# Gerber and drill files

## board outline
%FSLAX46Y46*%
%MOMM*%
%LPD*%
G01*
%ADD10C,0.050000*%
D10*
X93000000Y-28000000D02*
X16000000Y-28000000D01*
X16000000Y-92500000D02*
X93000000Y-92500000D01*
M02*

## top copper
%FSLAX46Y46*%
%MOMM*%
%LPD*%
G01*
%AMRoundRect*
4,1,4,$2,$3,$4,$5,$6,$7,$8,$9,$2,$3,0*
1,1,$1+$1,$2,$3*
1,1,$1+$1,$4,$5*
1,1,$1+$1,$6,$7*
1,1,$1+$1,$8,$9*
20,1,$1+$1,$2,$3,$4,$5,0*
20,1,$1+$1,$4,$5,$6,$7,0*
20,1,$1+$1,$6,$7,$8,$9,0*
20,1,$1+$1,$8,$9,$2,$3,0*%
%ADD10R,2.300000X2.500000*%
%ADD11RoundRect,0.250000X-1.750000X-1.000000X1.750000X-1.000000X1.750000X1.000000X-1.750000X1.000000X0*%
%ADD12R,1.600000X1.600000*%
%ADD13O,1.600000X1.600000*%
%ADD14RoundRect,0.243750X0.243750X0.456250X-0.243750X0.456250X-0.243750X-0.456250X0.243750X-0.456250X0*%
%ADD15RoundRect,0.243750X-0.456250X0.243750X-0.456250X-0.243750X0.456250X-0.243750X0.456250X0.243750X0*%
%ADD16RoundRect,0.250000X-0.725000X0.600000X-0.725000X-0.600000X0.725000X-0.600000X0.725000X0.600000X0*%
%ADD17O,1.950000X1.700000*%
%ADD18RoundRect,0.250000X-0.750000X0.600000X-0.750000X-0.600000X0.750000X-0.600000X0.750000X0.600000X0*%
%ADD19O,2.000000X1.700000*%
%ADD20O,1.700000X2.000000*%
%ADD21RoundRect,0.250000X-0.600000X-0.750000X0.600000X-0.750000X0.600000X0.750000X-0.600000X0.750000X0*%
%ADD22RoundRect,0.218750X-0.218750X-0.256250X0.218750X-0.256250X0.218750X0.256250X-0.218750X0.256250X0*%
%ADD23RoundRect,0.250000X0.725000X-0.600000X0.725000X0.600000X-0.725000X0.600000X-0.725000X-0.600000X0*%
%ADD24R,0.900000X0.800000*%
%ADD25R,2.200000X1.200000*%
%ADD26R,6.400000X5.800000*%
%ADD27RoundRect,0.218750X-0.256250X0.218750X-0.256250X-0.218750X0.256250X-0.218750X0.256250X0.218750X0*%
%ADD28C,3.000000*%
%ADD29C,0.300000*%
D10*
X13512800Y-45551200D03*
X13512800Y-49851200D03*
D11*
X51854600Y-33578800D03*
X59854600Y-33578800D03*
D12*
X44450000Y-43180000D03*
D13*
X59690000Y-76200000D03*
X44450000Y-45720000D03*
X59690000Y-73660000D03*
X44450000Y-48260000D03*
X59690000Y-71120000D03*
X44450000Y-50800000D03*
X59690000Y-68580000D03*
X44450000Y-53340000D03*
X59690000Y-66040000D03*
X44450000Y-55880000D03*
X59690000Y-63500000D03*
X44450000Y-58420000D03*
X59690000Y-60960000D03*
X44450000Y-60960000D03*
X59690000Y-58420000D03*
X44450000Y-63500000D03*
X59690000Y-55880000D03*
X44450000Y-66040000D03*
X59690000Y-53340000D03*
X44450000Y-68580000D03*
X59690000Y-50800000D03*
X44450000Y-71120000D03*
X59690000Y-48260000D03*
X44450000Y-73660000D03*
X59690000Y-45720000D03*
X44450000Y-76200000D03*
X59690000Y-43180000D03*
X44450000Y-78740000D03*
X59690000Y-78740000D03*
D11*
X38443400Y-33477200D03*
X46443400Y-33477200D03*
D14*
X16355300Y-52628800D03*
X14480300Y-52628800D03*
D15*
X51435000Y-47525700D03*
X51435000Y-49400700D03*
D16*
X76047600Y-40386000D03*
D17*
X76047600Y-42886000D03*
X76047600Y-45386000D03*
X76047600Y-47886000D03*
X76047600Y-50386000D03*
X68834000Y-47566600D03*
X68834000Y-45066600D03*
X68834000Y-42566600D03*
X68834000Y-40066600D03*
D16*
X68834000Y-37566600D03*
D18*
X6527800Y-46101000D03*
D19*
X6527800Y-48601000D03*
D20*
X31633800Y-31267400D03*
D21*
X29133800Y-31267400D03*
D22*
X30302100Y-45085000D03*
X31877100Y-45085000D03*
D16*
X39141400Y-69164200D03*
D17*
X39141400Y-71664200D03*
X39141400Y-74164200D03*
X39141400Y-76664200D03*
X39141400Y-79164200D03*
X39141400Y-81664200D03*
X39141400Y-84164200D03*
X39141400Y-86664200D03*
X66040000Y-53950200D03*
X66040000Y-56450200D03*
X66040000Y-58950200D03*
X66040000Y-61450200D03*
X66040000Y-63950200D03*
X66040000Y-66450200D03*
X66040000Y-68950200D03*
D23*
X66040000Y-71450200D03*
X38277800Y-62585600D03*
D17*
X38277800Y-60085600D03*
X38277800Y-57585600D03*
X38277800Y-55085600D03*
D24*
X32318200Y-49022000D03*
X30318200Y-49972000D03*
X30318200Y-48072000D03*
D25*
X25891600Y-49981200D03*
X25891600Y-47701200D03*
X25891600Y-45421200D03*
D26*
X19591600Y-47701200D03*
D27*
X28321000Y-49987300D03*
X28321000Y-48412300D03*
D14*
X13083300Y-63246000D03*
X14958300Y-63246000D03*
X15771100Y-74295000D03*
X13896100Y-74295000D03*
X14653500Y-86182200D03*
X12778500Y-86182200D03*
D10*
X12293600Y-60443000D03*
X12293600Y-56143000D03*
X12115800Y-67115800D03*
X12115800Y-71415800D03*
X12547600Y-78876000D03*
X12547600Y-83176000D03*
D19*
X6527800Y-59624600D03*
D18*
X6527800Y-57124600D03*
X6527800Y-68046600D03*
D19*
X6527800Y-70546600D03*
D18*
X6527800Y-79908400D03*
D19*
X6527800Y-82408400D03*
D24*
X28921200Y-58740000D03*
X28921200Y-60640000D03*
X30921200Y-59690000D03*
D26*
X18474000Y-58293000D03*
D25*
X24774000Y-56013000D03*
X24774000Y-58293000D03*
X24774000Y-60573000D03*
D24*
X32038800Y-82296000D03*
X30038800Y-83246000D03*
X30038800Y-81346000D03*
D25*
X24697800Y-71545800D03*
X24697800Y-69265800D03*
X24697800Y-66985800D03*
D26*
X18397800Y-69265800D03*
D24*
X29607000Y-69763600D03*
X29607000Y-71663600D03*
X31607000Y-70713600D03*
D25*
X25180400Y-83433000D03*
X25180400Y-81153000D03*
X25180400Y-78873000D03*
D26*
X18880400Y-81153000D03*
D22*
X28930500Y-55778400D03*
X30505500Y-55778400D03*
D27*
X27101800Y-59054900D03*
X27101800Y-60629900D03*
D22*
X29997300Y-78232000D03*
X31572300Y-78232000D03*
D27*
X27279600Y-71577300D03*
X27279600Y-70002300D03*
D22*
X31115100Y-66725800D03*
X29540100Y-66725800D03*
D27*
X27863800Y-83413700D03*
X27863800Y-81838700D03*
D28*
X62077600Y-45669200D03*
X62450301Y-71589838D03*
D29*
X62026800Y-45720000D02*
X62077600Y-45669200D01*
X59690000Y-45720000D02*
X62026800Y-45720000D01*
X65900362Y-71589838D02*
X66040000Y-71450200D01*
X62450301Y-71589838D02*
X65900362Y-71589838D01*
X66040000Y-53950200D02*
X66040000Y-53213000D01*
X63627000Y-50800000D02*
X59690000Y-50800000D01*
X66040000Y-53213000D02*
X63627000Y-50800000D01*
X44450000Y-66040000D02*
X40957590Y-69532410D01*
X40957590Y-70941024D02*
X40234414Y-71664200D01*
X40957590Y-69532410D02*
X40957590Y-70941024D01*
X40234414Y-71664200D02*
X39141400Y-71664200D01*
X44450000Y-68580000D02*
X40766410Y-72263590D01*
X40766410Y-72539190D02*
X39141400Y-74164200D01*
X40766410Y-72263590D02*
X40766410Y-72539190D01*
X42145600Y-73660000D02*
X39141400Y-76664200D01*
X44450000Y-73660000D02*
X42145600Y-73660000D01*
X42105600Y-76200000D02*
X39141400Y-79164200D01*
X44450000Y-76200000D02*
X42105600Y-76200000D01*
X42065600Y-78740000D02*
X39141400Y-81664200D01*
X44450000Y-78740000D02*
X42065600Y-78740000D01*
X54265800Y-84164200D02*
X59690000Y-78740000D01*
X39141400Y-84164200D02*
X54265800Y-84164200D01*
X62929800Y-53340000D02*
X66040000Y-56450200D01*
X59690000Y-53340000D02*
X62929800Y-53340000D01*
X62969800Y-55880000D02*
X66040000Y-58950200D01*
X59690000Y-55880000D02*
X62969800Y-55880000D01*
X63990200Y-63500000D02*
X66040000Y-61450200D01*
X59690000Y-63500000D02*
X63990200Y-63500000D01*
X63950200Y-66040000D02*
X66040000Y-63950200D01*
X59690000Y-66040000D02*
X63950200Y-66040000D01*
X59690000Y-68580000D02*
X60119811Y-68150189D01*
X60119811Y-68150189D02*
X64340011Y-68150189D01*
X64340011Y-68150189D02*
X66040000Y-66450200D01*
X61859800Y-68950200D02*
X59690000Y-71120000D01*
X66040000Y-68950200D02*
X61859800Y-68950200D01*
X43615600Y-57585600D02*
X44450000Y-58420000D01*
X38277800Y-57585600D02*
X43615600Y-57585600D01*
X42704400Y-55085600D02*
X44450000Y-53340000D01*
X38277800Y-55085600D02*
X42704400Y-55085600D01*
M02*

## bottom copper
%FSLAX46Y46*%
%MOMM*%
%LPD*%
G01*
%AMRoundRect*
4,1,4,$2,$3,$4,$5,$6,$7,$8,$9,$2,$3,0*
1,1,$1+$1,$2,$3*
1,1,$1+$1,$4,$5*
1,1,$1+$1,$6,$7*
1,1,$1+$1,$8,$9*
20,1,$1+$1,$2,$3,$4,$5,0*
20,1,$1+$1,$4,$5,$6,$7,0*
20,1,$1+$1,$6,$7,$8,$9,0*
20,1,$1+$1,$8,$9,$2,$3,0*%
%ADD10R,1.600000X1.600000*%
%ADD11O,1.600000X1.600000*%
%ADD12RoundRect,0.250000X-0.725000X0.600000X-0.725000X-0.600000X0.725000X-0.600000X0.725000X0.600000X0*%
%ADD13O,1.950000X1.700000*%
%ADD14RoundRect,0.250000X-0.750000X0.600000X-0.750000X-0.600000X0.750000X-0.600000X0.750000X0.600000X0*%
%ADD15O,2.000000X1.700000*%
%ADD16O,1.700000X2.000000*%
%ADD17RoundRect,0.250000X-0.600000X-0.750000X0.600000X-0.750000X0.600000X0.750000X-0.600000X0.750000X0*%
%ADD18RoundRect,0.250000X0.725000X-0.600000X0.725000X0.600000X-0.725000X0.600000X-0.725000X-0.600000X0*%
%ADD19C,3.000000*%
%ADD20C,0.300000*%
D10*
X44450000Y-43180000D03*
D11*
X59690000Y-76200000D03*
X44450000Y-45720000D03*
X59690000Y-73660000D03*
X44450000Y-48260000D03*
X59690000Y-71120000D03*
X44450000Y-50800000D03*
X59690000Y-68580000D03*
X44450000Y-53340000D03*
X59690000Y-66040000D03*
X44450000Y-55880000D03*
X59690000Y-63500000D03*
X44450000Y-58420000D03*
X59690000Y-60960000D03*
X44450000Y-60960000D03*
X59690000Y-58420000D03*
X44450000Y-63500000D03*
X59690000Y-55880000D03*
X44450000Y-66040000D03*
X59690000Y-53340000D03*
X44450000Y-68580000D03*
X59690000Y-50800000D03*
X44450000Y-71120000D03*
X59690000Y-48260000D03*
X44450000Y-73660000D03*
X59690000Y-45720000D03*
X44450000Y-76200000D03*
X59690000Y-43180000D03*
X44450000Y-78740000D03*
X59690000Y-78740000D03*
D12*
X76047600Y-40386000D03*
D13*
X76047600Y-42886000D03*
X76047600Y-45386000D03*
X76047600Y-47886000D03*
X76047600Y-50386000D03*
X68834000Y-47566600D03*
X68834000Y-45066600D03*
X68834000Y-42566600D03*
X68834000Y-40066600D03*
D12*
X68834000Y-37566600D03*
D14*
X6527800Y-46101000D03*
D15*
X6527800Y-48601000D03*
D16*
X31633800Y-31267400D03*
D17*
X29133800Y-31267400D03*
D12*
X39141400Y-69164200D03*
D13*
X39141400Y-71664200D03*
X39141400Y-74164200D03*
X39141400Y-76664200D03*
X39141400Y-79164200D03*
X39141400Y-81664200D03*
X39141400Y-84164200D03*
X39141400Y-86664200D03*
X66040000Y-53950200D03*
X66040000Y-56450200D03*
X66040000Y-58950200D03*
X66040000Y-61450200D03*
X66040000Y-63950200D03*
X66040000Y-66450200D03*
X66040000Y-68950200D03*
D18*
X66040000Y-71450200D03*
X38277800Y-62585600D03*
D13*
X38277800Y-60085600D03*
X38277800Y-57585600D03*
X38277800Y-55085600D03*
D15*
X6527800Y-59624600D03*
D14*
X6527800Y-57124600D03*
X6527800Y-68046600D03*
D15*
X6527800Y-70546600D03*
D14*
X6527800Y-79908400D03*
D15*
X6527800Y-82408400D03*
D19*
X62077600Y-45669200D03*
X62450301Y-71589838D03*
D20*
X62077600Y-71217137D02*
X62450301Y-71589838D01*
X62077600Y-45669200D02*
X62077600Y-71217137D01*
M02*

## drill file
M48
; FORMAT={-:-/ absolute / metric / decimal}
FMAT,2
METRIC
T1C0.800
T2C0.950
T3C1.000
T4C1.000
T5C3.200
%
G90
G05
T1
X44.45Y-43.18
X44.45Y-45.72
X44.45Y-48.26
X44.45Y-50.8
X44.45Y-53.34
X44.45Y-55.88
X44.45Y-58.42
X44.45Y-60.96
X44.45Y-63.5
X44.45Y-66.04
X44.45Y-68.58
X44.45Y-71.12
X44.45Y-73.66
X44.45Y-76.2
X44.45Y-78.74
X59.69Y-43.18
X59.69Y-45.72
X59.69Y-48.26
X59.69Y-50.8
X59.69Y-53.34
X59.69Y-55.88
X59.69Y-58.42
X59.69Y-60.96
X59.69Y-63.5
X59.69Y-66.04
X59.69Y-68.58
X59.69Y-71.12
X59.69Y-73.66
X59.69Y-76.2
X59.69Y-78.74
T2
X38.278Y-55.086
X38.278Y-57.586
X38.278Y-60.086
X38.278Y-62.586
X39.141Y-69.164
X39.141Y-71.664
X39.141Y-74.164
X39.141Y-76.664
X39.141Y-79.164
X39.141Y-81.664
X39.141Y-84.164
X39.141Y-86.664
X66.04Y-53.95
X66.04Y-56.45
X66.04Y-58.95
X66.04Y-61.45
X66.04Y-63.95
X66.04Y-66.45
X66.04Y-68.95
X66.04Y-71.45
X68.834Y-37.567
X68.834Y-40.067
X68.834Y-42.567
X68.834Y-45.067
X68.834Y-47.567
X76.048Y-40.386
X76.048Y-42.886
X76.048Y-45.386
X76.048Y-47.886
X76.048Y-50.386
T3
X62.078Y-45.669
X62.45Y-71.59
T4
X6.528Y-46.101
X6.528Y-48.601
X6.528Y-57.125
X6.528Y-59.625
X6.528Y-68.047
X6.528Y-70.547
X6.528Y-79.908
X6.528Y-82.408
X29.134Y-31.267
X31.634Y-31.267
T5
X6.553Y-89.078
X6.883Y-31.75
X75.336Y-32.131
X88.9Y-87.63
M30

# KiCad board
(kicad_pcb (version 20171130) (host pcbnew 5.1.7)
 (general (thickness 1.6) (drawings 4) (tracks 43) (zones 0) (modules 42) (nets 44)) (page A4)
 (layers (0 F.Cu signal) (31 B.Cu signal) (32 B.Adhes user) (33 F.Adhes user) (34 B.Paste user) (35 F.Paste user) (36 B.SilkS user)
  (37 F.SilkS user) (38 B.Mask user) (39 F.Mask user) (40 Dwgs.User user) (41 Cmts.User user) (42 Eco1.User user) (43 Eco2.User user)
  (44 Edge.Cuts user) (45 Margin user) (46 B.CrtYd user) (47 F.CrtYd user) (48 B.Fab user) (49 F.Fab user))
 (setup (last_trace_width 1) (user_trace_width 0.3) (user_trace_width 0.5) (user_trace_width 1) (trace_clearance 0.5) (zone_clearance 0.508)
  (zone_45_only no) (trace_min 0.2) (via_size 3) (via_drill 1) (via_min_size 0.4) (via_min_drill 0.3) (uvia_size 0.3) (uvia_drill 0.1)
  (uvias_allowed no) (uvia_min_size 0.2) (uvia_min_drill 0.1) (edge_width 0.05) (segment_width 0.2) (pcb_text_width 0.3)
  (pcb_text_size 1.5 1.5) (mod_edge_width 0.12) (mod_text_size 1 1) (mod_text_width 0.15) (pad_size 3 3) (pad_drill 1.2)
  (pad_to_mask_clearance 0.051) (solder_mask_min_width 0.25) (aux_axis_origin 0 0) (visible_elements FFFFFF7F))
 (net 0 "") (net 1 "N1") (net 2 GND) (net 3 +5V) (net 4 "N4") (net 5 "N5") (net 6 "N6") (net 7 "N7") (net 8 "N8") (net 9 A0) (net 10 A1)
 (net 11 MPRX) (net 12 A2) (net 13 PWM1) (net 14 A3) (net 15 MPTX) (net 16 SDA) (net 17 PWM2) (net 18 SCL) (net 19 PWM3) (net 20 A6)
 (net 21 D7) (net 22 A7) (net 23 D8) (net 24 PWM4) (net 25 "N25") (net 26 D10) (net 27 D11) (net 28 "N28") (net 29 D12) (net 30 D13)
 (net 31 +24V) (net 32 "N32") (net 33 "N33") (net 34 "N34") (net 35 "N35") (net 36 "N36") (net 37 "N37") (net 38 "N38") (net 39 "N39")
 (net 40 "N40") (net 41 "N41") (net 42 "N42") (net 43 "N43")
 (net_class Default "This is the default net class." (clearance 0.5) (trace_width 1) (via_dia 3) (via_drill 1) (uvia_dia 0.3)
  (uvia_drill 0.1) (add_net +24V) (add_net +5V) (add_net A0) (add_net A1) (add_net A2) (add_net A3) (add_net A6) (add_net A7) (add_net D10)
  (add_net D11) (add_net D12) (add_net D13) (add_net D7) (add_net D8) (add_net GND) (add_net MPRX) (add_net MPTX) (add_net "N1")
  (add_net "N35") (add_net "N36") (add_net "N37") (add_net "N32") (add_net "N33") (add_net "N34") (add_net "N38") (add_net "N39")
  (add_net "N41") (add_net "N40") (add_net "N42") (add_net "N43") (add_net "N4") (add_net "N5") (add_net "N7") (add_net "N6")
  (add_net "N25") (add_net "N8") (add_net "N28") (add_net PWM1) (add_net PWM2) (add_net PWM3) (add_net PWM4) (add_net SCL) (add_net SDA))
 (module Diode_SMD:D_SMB (layer F.Cu) (at 13.5128 47.7012 270)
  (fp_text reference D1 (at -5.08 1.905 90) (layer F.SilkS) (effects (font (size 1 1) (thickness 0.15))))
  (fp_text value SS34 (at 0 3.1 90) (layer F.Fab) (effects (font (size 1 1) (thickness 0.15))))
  (pad 1 smd rect (at -2.15 0 270) (size 2.5 2.3) (layers F.Cu F.Paste F.Mask) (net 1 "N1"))
  (pad 2 smd rect (at 2.15 0 270) (size 2.5 2.3) (layers F.Cu F.Paste F.Mask) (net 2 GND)))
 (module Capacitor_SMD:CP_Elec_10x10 (layer F.Cu) (at 55.8546 33.5788)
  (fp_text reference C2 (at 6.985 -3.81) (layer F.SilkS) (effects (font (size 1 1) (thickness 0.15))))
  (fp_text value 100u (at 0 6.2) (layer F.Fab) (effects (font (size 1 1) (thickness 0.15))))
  (pad 1 smd roundrect (at -4 0) (size 4 2.5) (layers F.Cu F.Paste F.Mask) (roundrect_rratio 0.1) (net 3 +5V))
  (pad 2 smd roundrect (at 4 0) (size 4 2.5) (layers F.Cu F.Paste F.Mask) (roundrect_rratio 0.1) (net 2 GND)))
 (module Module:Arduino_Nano (layer F.Cu) (at 44.45 43.18)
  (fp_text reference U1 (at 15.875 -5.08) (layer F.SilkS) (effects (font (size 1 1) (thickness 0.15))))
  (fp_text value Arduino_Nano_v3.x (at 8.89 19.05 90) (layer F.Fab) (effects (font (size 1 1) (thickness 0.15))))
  (pad 1 thru_hole rect (at 0 0) (size 1.6 1.6) (drill 0.8) (layers *.Cu *.Mask) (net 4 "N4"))
  (pad 17 thru_hole oval (at 15.24 33.02) (size 1.6 1.6) (drill 0.8) (layers *.Cu *.Mask) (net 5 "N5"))
  (pad 2 thru_hole oval (at 0 2.54) (size 1.6 1.6) (drill 0.8) (layers *.Cu *.Mask) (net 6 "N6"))
  (pad 18 thru_hole oval (at 15.24 30.48) (size 1.6 1.6) (drill 0.8) (layers *.Cu *.Mask) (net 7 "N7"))
  (pad 3 thru_hole oval (at 0 5.08) (size 1.6 1.6) (drill 0.8) (layers *.Cu *.Mask) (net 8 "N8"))
  (pad 19 thru_hole oval (at 15.24 27.94) (size 1.6 1.6) (drill 0.8) (layers *.Cu *.Mask) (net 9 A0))
  (pad 4 thru_hole oval (at 0 7.62) (size 1.6 1.6) (drill 0.8) (layers *.Cu *.Mask) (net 2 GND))
  (pad 20 thru_hole oval (at 15.24 25.4) (size 1.6 1.6) (drill 0.8) (layers *.Cu *.Mask) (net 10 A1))
  (pad 5 thru_hole oval (at 0 10.16) (size 1.6 1.6) (drill 0.8) (layers *.Cu *.Mask) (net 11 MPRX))
  (pad 21 thru_hole oval (at 15.24 22.86) (size 1.6 1.6) (drill 0.8) (layers *.Cu *.Mask) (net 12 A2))
  (pad 6 thru_hole oval (at 0 12.7) (size 1.6 1.6) (drill 0.8) (layers *.Cu *.Mask) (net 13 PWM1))
  (pad 22 thru_hole oval (at 15.24 20.32) (size 1.6 1.6) (drill 0.8) (layers *.Cu *.Mask) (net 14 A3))
  (pad 7 thru_hole oval (at 0 15.24) (size 1.6 1.6) (drill 0.8) (layers *.Cu *.Mask) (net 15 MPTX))
  (pad 23 thru_hole oval (at 15.24 17.78) (size 1.6 1.6) (drill 0.8) (layers *.Cu *.Mask) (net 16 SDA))
  (pad 8 thru_hole oval (at 0 17.78) (size 1.6 1.6) (drill 0.8) (layers *.Cu *.Mask) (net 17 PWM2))
  (pad 24 thru_hole oval (at 15.24 15.24) (size 1.6 1.6) (drill 0.8) (layers *.Cu *.Mask) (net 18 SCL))
  (pad 9 thru_hole oval (at 0 20.32) (size 1.6 1.6) (drill 0.8) (layers *.Cu *.Mask) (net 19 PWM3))
  (pad 25 thru_hole oval (at 15.24 12.7) (size 1.6 1.6) (drill 0.8) (layers *.Cu *.Mask) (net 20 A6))
  (pad 10 thru_hole oval (at 0 22.86) (size 1.6 1.6) (drill 0.8) (layers *.Cu *.Mask) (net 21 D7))
  (pad 26 thru_hole oval (at 15.24 10.16) (size 1.6 1.6) (drill 0.8) (layers *.Cu *.Mask) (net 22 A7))
  (pad 11 thru_hole oval (at 0 25.4) (size 1.6 1.6) (drill 0.8) (layers *.Cu *.Mask) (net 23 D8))
  (pad 27 thru_hole oval (at 15.24 7.62) (size 1.6 1.6) (drill 0.8) (layers *.Cu *.Mask) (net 3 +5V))
  (pad 12 thru_hole oval (at 0 27.94) (size 1.6 1.6) (drill 0.8) (layers *.Cu *.Mask) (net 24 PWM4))
  (pad 28 thru_hole oval (at 15.24 5.08) (size 1.6 1.6) (drill 0.8) (layers *.Cu *.Mask) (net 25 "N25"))
  (pad 13 thru_hole oval (at 0 30.48) (size 1.6 1.6) (drill 0.8) (layers *.Cu *.Mask) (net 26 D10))
  (pad 29 thru_hole oval (at 15.24 2.54) (size 1.6 1.6) (drill 0.8) (layers *.Cu *.Mask) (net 2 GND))
  (pad 14 thru_hole oval (at 0 33.02) (size 1.6 1.6) (drill 0.8) (layers *.Cu *.Mask) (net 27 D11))
  (pad 30 thru_hole oval (at 15.24 0) (size 1.6 1.6) (drill 0.8) (layers *.Cu *.Mask) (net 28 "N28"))
  (pad 15 thru_hole oval (at 0 35.56) (size 1.6 1.6) (drill 0.8) (layers *.Cu *.Mask) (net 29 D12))
  (pad 16 thru_hole oval (at 15.24 35.56) (size 1.6 1.6) (drill 0.8) (layers *.Cu *.Mask) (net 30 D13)))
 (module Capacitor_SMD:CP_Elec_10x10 (layer F.Cu) (at 42.4434 33.4772)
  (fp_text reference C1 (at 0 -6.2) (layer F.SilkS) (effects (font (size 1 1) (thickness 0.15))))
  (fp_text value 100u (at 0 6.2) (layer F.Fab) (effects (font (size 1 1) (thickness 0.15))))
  (pad 1 smd roundrect (at -4 0) (size 4 2.5) (layers F.Cu F.Paste F.Mask) (roundrect_rratio 0.1) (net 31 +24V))
  (pad 2 smd roundrect (at 4 0) (size 4 2.5) (layers F.Cu F.Paste F.Mask) (roundrect_rratio 0.1) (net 2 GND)))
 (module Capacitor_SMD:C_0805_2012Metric (layer F.Cu) (at 15.4178 52.6288 180)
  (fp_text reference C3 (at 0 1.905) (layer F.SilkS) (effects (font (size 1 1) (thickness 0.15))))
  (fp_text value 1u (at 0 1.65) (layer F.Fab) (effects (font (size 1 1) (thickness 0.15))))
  (pad 1 smd roundrect (at -0.9375 0 180) (size 0.975 1.4) (layers F.Cu F.Paste F.Mask) (roundrect_rratio 0.25) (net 31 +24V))
  (pad 2 smd roundrect (at 0.9375 0 180) (size 0.975 1.4) (layers F.Cu F.Paste F.Mask) (roundrect_rratio 0.25) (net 2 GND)))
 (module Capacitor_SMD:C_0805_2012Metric (layer F.Cu) (at 51.435 48.4632 270)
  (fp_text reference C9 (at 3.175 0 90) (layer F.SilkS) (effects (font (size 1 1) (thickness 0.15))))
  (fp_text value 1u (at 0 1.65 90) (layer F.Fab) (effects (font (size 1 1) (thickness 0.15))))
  (pad 1 smd roundrect (at -0.9375 0 270) (size 0.975 1.4) (layers F.Cu F.Paste F.Mask) (roundrect_rratio 0.25) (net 2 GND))
  (pad 2 smd roundrect (at 0.9375 0 270) (size 0.975 1.4) (layers F.Cu F.Paste F.Mask) (roundrect_rratio 0.25) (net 3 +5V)))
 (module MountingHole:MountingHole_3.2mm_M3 (layer F.Cu) (at 88.9 87.63)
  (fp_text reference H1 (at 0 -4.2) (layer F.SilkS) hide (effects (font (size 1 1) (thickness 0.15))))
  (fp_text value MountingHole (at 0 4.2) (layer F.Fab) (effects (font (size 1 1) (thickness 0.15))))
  (pad 1 np_thru_hole circle (at 0 0) (size 3.2 3.2) (drill 3.2) (layers *.Cu *.Mask)))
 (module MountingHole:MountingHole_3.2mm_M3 (layer F.Cu) (at 6.5532 89.0778)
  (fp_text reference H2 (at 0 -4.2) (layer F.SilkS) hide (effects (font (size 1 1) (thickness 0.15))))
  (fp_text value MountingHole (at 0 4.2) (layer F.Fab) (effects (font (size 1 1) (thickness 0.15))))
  (pad 1 np_thru_hole circle (at 0 0) (size 3.2 3.2) (drill 3.2) (layers *.Cu *.Mask)))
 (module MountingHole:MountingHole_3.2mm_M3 (layer F.Cu) (at 75.3364 32.131)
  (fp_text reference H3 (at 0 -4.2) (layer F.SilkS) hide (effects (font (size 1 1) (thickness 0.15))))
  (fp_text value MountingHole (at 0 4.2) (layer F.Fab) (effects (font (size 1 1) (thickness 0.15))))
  (pad 1 np_thru_hole circle (at 0 0) (size 3.2 3.2) (drill 3.2) (layers *.Cu *.Mask)))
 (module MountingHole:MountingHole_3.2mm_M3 (layer F.Cu) (at 6.8834 31.75)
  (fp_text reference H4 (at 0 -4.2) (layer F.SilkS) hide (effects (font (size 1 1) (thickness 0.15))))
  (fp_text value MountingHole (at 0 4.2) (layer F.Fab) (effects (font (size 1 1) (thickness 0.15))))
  (pad 1 np_thru_hole circle (at 0 0) (size 3.2 3.2) (drill 3.2) (layers *.Cu *.Mask)))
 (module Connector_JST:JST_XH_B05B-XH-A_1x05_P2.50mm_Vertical (layer F.Cu) (at 76.0476 40.386 270)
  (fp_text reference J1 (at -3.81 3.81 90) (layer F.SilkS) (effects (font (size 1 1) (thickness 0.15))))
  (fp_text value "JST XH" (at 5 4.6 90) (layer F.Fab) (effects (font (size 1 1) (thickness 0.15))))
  (pad 1 thru_hole roundrect (at 0 0 270) (size 1.7 1.95) (drill 0.95) (layers *.Cu *.Mask) (roundrect_rratio 0.147059) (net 3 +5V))
  (pad 2 thru_hole oval (at 2.5 0 270) (size 1.7 1.95) (drill 0.95) (layers *.Cu *.Mask) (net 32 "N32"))
  (pad 3 thru_hole oval (at 5 0 270) (size 1.7 1.95) (drill 0.95) (layers *.Cu *.Mask) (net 16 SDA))
  (pad 4 thru_hole oval (at 7.5 0 270) (size 1.7 1.95) (drill 0.95) (layers *.Cu *.Mask) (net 18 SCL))
  (pad 5 thru_hole oval (at 10 0 270) (size 1.7 1.95) (drill 0.95) (layers *.Cu *.Mask) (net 2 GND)))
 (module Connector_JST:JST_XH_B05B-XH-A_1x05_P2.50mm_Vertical (layer F.Cu) (at 68.834 37.5666 270)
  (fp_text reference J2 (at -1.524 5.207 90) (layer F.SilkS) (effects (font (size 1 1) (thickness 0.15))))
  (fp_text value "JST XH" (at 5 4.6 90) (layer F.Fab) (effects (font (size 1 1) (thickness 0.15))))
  (pad 5 thru_hole oval (at 10 0 270) (size 1.7 1.95) (drill 0.95) (layers *.Cu *.Mask) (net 2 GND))
  (pad 4 thru_hole oval (at 7.5 0 270) (size 1.7 1.95) (drill 0.95) (layers *.Cu *.Mask) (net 18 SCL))
  (pad 3 thru_hole oval (at 5 0 270) (size 1.7 1.95) (drill 0.95) (layers *.Cu *.Mask) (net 16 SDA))
  (pad 2 thru_hole oval (at 2.5 0 270) (size 1.7 1.95) (drill 0.95) (layers *.Cu *.Mask) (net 32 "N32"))
  (pad 1 thru_hole roundrect (at 0 0 270) (size 1.7 1.95) (drill 0.95) (layers *.Cu *.Mask) (roundrect_rratio 0.147059) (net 3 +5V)))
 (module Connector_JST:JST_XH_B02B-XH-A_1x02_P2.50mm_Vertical (layer F.Cu) (at 6.5278 46.101 270)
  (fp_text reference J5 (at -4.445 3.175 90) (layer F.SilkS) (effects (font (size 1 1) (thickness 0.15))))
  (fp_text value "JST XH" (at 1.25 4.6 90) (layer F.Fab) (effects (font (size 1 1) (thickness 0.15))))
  (pad 1 thru_hole roundrect (at 0 0 270) (size 1.7 2) (drill 1) (layers *.Cu *.Mask) (roundrect_rratio 0.147059) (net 1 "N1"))
  (pad 2 thru_hole oval (at 2.5 0 270) (size 1.7 2) (drill 1) (layers *.Cu *.Mask) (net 2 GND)))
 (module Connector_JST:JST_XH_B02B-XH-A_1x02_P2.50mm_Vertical (layer F.Cu) (at 29.1338 31.2674)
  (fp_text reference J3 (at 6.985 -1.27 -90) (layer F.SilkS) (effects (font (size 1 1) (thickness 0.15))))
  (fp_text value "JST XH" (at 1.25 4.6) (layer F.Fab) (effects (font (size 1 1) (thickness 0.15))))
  (pad 2 thru_hole oval (at 2.5 0) (size 1.7 2) (drill 1) (layers *.Cu *.Mask) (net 2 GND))
  (pad 1 thru_hole roundrect (at 0 0) (size 1.7 2) (drill 1) (layers *.Cu *.Mask) (roundrect_rratio 0.147059) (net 31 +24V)))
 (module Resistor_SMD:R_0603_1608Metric (layer F.Cu) (at 31.0896 45.085)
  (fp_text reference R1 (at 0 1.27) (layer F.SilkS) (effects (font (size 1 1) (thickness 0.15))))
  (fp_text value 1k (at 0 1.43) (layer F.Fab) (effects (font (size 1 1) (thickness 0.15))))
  (pad 1 smd roundrect (at -0.7875 0) (size 0.875 0.95) (layers F.Cu F.Paste F.Mask) (roundrect_rratio 0.25) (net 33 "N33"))
  (pad 2 smd roundrect (at 0.7875 0) (size 0.875 0.95) (layers F.Cu F.Paste F.Mask) (roundrect_rratio 0.25) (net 13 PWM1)))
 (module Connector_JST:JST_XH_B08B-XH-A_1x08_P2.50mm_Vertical (layer F.Cu) (at 39.1414 69.1642 270)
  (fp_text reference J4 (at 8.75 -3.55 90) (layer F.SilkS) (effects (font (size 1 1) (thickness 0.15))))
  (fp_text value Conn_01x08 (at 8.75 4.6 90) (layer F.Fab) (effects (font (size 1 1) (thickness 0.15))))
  (pad 1 thru_hole roundrect (at 0 0 270) (size 1.7 1.95) (drill 0.95) (layers *.Cu *.Mask) (roundrect_rratio 0.147059) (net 2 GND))
  (pad 2 thru_hole oval (at 2.5 0 270) (size 1.7 1.95) (drill 0.95) (layers *.Cu *.Mask) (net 21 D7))
  (pad 3 thru_hole oval (at 5 0 270) (size 1.7 1.95) (drill 0.95) (layers *.Cu *.Mask) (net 23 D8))
  (pad 4 thru_hole oval (at 7.5 0 270) (size 1.7 1.95) (drill 0.95) (layers *.Cu *.Mask) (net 26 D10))
  (pad 5 thru_hole oval (at 10 0 270) (size 1.7 1.95) (drill 0.95) (layers *.Cu *.Mask) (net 27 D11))
  (pad 6 thru_hole oval (at 12.5 0 270) (size 1.7 1.95) (drill 0.95) (layers *.Cu *.Mask) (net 29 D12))
  (pad 7 thru_hole oval (at 15 0 270) (size 1.7 1.95) (drill 0.95) (layers *.Cu *.Mask) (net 30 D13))
  (pad 8 thru_hole oval (at 17.5 0 270) (size 1.7 1.95) (drill 0.95) (layers *.Cu *.Mask) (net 3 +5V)))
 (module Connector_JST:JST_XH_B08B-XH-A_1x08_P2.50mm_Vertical (layer F.Cu) (at 66.04 71.4502 90)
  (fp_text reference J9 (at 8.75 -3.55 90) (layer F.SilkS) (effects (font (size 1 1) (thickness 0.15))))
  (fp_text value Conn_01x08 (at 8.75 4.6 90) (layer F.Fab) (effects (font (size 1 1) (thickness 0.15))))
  (pad 8 thru_hole oval (at 17.5 0 90) (size 1.7 1.95) (drill 0.95) (layers *.Cu *.Mask) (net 3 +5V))
  (pad 7 thru_hole oval (at 15 0 90) (size 1.7 1.95) (drill 0.95) (layers *.Cu *.Mask) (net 22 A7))
  (pad 6 thru_hole oval (at 12.5 0 90) (size 1.7 1.95) (drill 0.95) (layers *.Cu *.Mask) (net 20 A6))
  (pad 5 thru_hole oval (at 10 0 90) (size 1.7 1.95) (drill 0.95) (layers *.Cu *.Mask) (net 14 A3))
  (pad 4 thru_hole oval (at 7.5 0 90) (size 1.7 1.95) (drill 0.95) (layers *.Cu *.Mask) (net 12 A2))
  (pad 3 thru_hole oval (at 5 0 90) (size 1.7 1.95) (drill 0.95) (layers *.Cu *.Mask) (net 10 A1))
  (pad 2 thru_hole oval (at 2.5 0 90) (size 1.7 1.95) (drill 0.95) (layers *.Cu *.Mask) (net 9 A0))
  (pad 1 thru_hole roundrect (at 0 0 90) (size 1.7 1.95) (drill 0.95) (layers *.Cu *.Mask) (roundrect_rratio 0.147059) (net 2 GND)))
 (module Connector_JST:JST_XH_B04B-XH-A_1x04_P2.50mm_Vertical (layer F.Cu) (at 38.2778 62.5856 90)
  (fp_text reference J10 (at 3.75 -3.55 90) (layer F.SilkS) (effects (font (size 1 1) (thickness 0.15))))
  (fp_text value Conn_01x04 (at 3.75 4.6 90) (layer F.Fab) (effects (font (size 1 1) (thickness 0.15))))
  (pad 1 thru_hole roundrect (at 0 0 90) (size 1.7 1.95) (drill 0.95) (layers *.Cu *.Mask) (roundrect_rratio 0.147059) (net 2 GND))
  (pad 2 thru_hole oval (at 2.5 0 90) (size 1.7 1.95) (drill 0.95) (layers *.Cu *.Mask) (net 3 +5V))
  (pad 3 thru_hole oval (at 5 0 90) (size 1.7 1.95) (drill 0.95) (layers *.Cu *.Mask) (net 15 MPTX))
  (pad 4 thru_hole oval (at 7.5 0 90) (size 1.7 1.95) (drill 0.95) (layers *.Cu *.Mask) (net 11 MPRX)))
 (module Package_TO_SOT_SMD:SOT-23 (layer F.Cu) (at 31.3182 49.022)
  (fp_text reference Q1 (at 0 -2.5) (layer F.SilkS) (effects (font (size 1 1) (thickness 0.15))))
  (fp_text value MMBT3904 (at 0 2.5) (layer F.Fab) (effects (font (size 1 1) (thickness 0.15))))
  (pad 3 smd rect (at 1 0) (size 0.9 0.8) (layers F.Cu F.Paste F.Mask) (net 2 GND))
  (pad 2 smd rect (at -1 0.95) (size 0.9 0.8) (layers F.Cu F.Paste F.Mask) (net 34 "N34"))
  (pad 1 smd rect (at -1 -0.95) (size 0.9 0.8) (layers F.Cu F.Paste F.Mask) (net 33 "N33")))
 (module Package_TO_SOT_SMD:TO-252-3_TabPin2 (layer F.Cu) (at 21.6916 47.7012 180)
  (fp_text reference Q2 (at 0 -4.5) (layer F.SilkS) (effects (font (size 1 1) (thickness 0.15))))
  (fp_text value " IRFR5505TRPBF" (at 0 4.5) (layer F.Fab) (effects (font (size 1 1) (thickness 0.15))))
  (pad 1 smd rect (at -4.2 -2.28 180) (size 2.2 1.2) (layers F.Cu F.Paste F.Mask) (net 34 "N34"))
  (pad 2 smd rect (at -4.2 0 180) (size 2.2 1.2) (layers F.Cu F.Paste F.Mask) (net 31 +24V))
  (pad 3 smd rect (at -4.2 2.28 180) (size 2.2 1.2) (layers F.Cu F.Paste F.Mask) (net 1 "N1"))
  (pad 2 smd rect (at 2.1 0 180) (size 6.4 5.8) (layers F.Cu F.Mask) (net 31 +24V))
  (pad "" smd rect (at 3.775 1.525 180) (size 3.05 2.75) (layers F.Paste))
  (pad "" smd rect (at 0.425 -1.525 180) (size 3.05 2.75) (layers F.Paste))
  (pad "" smd rect (at 3.775 -1.525 180) (size 3.05 2.75) (layers F.Paste))
  (pad "" smd rect (at 0.425 1.525 180) (size 3.05 2.75) (layers F.Paste)))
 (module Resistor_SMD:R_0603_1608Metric (layer F.Cu) (at 28.321 49.1998 270)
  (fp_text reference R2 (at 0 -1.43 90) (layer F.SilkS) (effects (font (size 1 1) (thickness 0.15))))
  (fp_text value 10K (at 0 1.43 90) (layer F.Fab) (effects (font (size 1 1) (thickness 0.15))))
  (pad 2 smd roundrect (at 0.7875 0 270) (size 0.875 0.95) (layers F.Cu F.Paste F.Mask) (roundrect_rratio 0.25) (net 34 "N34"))
  (pad 1 smd roundrect (at -0.7875 0 270) (size 0.875 0.95) (layers F.Cu F.Paste F.Mask) (roundrect_rratio 0.25) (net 31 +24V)))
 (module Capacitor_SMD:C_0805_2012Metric (layer F.Cu) (at 14.0208 63.246 180)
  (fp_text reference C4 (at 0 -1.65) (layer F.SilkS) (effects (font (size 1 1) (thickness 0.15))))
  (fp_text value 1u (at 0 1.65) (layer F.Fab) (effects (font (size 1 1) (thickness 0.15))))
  (pad 2 smd roundrect (at 0.9375 0 180) (size 0.975 1.4) (layers F.Cu F.Paste F.Mask) (roundrect_rratio 0.25) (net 2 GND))
  (pad 1 smd roundrect (at -0.9375 0 180) (size 0.975 1.4) (layers F.Cu F.Paste F.Mask) (roundrect_rratio 0.25) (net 31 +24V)))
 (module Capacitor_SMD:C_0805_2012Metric (layer F.Cu) (at 14.8336 74.295 180)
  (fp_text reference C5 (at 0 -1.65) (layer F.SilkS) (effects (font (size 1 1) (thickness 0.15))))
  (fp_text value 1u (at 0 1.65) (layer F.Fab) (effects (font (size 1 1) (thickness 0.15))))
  (pad 1 smd roundrect (at -0.9375 0 180) (size 0.975 1.4) (layers F.Cu F.Paste F.Mask) (roundrect_rratio 0.25) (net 31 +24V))
  (pad 2 smd roundrect (at 0.9375 0 180) (size 0.975 1.4) (layers F.Cu F.Paste F.Mask) (roundrect_rratio 0.25) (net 2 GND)))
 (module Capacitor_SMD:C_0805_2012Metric (layer F.Cu) (at 13.716 86.1822 180)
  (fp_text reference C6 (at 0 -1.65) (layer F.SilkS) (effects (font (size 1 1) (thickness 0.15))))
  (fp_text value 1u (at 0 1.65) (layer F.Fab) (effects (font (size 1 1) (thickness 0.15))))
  (pad 1 smd roundrect (at -0.9375 0 180) (size 0.975 1.4) (layers F.Cu F.Paste F.Mask) (roundrect_rratio 0.25) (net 31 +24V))
  (pad 2 smd roundrect (at 0.9375 0 180) (size 0.975 1.4) (layers F.Cu F.Paste F.Mask) (roundrect_rratio 0.25) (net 2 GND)))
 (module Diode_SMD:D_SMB (layer F.Cu) (at 12.2936 58.293 270)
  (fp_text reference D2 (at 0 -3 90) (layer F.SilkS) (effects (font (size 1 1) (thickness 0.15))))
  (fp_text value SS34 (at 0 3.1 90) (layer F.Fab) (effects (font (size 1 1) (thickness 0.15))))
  (pad 2 smd rect (at 2.15 0 270) (size 2.5 2.3) (layers F.Cu F.Paste F.Mask) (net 2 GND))
  (pad 1 smd rect (at -2.15 0 270) (size 2.5 2.3) (layers F.Cu F.Paste F.Mask) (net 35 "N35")))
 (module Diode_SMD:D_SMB (layer F.Cu) (at 12.1158 69.2658 270)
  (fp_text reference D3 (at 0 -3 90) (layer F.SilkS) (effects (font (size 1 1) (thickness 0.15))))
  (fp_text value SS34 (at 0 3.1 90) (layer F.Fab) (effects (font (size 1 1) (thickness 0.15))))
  (pad 1 smd rect (at -2.15 0 270) (size 2.5 2.3) (layers F.Cu F.Paste F.Mask) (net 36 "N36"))
  (pad 2 smd rect (at 2.15 0 270) (size 2.5 2.3) (layers F.Cu F.Paste F.Mask) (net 2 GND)))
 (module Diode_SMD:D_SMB (layer F.Cu) (at 12.5476 81.026 270)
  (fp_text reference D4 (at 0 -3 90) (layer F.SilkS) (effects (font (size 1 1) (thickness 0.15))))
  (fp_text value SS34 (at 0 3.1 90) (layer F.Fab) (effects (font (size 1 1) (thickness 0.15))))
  (pad 1 smd rect (at -2.15 0 270) (size 2.5 2.3) (layers F.Cu F.Paste F.Mask) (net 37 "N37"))
  (pad 2 smd rect (at 2.15 0 270) (size 2.5 2.3) (layers F.Cu F.Paste F.Mask) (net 2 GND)))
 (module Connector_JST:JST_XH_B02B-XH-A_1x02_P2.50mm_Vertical (layer F.Cu) (at 6.5278 57.1246 270)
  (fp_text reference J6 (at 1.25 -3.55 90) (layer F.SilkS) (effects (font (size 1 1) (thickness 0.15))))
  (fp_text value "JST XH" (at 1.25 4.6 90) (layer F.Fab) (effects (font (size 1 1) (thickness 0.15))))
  (pad 2 thru_hole oval (at 2.5 0 270) (size 1.7 2) (drill 1) (layers *.Cu *.Mask) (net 2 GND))
  (pad 1 thru_hole roundrect (at 0 0 270) (size 1.7 2) (drill 1) (layers *.Cu *.Mask) (roundrect_rratio 0.147059) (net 35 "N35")))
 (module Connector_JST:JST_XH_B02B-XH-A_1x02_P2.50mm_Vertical (layer F.Cu) (at 6.5278 68.0466 270)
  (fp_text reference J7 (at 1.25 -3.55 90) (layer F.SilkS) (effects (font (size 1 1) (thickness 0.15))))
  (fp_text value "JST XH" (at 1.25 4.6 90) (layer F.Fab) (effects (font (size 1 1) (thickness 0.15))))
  (pad 1 thru_hole roundrect (at 0 0 270) (size 1.7 2) (drill 1) (layers *.Cu *.Mask) (roundrect_rratio 0.147059) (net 36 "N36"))
  (pad 2 thru_hole oval (at 2.5 0 270) (size 1.7 2) (drill 1) (layers *.Cu *.Mask) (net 2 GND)))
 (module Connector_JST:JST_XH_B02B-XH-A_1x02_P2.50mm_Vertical (layer F.Cu) (at 6.5278 79.9084 270)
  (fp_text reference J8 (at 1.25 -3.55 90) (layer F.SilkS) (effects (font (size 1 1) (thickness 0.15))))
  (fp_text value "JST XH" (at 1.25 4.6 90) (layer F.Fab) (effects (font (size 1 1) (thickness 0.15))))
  (pad 1 thru_hole roundrect (at 0 0 270) (size 1.7 2) (drill 1) (layers *.Cu *.Mask) (roundrect_rratio 0.147059) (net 37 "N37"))
  (pad 2 thru_hole oval (at 2.5 0 270) (size 1.7 2) (drill 1) (layers *.Cu *.Mask) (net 2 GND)))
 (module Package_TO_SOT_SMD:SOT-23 (layer F.Cu) (at 29.9212 59.69)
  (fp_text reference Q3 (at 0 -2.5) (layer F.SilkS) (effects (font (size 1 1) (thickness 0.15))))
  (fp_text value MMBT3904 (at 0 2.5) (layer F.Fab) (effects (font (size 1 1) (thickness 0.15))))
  (pad 1 smd rect (at -1 -0.95) (size 0.9 0.8) (layers F.Cu F.Paste F.Mask) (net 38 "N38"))
  (pad 2 smd rect (at -1 0.95) (size 0.9 0.8) (layers F.Cu F.Paste F.Mask) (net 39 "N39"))
  (pad 3 smd rect (at 1 0) (size 0.9 0.8) (layers F.Cu F.Paste F.Mask) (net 2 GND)))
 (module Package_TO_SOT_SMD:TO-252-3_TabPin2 (layer F.Cu) (at 20.574 58.293 180)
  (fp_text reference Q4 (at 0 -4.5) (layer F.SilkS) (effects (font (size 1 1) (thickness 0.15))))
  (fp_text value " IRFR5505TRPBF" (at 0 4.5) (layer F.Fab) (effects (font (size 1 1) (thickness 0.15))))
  (pad "" smd rect (at 0.425 1.525 180) (size 3.05 2.75) (layers F.Paste))
  (pad "" smd rect (at 3.775 -1.525 180) (size 3.05 2.75) (layers F.Paste))
  (pad "" smd rect (at 0.425 -1.525 180) (size 3.05 2.75) (layers F.Paste))
  (pad "" smd rect (at 3.775 1.525 180) (size 3.05 2.75) (layers F.Paste))
  (pad 2 smd rect (at 2.1 0 180) (size 6.4 5.8) (layers F.Cu F.Mask) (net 31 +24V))
  (pad 3 smd rect (at -4.2 2.28 180) (size 2.2 1.2) (layers F.Cu F.Paste F.Mask) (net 35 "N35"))
  (pad 2 smd rect (at -4.2 0 180) (size 2.2 1.2) (layers F.Cu F.Paste F.Mask) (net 31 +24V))
  (pad 1 smd rect (at -4.2 -2.28 180) (size 2.2 1.2) (layers F.Cu F.Paste F.Mask) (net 39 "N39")))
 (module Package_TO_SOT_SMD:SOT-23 (layer F.Cu) (at 31.0388 82.296)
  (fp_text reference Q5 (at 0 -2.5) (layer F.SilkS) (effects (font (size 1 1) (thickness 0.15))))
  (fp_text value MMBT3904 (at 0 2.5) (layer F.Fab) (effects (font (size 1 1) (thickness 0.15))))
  (pad 3 smd rect (at 1 0) (size 0.9 0.8) (layers F.Cu F.Paste F.Mask) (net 2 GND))
  (pad 2 smd rect (at -1 0.95) (size 0.9 0.8) (layers F.Cu F.Paste F.Mask) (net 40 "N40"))
  (pad 1 smd rect (at -1 -0.95) (size 0.9 0.8) (layers F.Cu F.Paste F.Mask) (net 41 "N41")))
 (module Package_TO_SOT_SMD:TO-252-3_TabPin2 (layer F.Cu) (at 20.4978 69.2658 180)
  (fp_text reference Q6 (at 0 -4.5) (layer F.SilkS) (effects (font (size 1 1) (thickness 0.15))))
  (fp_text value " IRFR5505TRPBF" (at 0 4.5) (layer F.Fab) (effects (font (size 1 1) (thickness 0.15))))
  (pad 1 smd rect (at -4.2 -2.28 180) (size 2.2 1.2) (layers F.Cu F.Paste F.Mask) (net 40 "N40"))
  (pad 2 smd rect (at -4.2 0 180) (size 2.2 1.2) (layers F.Cu F.Paste F.Mask) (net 31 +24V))
  (pad 3 smd rect (at -4.2 2.28 180) (size 2.2 1.2) (layers F.Cu F.Paste F.Mask) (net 36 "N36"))
  (pad 2 smd rect (at 2.1 0 180) (size 6.4 5.8) (layers F.Cu F.Mask) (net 31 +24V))
  (pad "" smd rect (at 3.775 1.525 180) (size 3.05 2.75) (layers F.Paste))
  (pad "" smd rect (at 0.425 -1.525 180) (size 3.05 2.75) (layers F.Paste))
  (pad "" smd rect (at 3.775 -1.525 180) (size 3.05 2.75) (layers F.Paste))
  (pad "" smd rect (at 0.425 1.525 180) (size 3.05 2.75) (layers F.Paste)))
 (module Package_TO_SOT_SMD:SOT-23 (layer F.Cu) (at 30.607 70.7136)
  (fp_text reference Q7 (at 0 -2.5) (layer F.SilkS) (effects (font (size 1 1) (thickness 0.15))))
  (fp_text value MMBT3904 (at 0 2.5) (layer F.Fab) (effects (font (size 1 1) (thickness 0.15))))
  (pad 1 smd rect (at -1 -0.95) (size 0.9 0.8) (layers F.Cu F.Paste F.Mask) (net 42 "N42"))
  (pad 2 smd rect (at -1 0.95) (size 0.9 0.8) (layers F.Cu F.Paste F.Mask) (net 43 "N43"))
  (pad 3 smd rect (at 1 0) (size 0.9 0.8) (layers F.Cu F.Paste F.Mask) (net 2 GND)))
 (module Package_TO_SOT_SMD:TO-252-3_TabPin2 (layer F.Cu) (at 20.9804 81.153 180)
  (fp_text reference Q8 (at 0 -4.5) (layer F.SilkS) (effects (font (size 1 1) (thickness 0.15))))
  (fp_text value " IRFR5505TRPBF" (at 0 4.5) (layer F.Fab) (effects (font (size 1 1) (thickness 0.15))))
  (pad 1 smd rect (at -4.2 -2.28 180) (size 2.2 1.2) (layers F.Cu F.Paste F.Mask) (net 43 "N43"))
  (pad 2 smd rect (at -4.2 0 180) (size 2.2 1.2) (layers F.Cu F.Paste F.Mask) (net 31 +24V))
  (pad 3 smd rect (at -4.2 2.28 180) (size 2.2 1.2) (layers F.Cu F.Paste F.Mask) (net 37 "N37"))
  (pad 2 smd rect (at 2.1 0 180) (size 6.4 5.8) (layers F.Cu F.Mask) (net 31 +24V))
  (pad "" smd rect (at 3.775 1.525 180) (size 3.05 2.75) (layers F.Paste))
  (pad "" smd rect (at 0.425 -1.525 180) (size 3.05 2.75) (layers F.Paste))
  (pad "" smd rect (at 3.775 -1.525 180) (size 3.05 2.75) (layers F.Paste))
  (pad "" smd rect (at 0.425 1.525 180) (size 3.05 2.75) (layers F.Paste)))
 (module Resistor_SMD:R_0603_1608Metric (layer F.Cu) (at 29.718 55.7784)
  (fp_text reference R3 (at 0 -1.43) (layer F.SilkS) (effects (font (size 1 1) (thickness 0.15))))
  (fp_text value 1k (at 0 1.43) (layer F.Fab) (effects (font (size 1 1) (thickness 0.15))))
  (pad 1 smd roundrect (at -0.7875 0) (size 0.875 0.95) (layers F.Cu F.Paste F.Mask) (roundrect_rratio 0.25) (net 38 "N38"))
  (pad 2 smd roundrect (at 0.7875 0) (size 0.875 0.95) (layers F.Cu F.Paste F.Mask) (roundrect_rratio 0.25) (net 17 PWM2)))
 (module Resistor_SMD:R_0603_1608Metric (layer F.Cu) (at 27.1018 59.8424 270)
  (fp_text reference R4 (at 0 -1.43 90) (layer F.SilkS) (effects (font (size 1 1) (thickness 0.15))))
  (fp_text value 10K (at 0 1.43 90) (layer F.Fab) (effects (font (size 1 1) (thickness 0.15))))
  (pad 1 smd roundrect (at -0.7875 0 270) (size 0.875 0.95) (layers F.Cu F.Paste F.Mask) (roundrect_rratio 0.25) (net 31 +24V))
  (pad 2 smd roundrect (at 0.7875 0 270) (size 0.875 0.95) (layers F.Cu F.Paste F.Mask) (roundrect_rratio 0.25) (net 39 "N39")))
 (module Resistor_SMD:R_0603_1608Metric (layer F.Cu) (at 30.7848 78.232)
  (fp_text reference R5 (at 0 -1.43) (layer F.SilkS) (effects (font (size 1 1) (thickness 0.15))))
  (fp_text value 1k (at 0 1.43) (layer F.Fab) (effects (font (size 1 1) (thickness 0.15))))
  (pad 1 smd roundrect (at -0.7875 0) (size 0.875 0.95) (layers F.Cu F.Paste F.Mask) (roundrect_rratio 0.25) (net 41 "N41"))
  (pad 2 smd roundrect (at 0.7875 0) (size 0.875 0.95) (layers F.Cu F.Paste F.Mask) (roundrect_rratio 0.25) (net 19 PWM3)))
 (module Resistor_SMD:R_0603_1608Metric (layer F.Cu) (at 27.2796 70.7898 270)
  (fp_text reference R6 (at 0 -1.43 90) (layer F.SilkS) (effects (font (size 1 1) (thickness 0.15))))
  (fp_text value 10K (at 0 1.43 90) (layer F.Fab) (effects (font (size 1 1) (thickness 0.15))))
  (pad 2 smd roundrect (at 0.7875 0 270) (size 0.875 0.95) (layers F.Cu F.Paste F.Mask) (roundrect_rratio 0.25) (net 40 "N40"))
  (pad 1 smd roundrect (at -0.7875 0 270) (size 0.875 0.95) (layers F.Cu F.Paste F.Mask) (roundrect_rratio 0.25) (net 31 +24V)))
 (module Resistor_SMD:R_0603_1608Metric (layer F.Cu) (at 30.3276 66.7258)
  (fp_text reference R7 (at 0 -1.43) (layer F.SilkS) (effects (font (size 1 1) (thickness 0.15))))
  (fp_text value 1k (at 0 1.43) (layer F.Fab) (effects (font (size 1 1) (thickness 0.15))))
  (pad 2 smd roundrect (at 0.7875 0) (size 0.875 0.95) (layers F.Cu F.Paste F.Mask) (roundrect_rratio 0.25) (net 24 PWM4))
  (pad 1 smd roundrect (at -0.7875 0) (size 0.875 0.95) (layers F.Cu F.Paste F.Mask) (roundrect_rratio 0.25) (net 42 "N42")))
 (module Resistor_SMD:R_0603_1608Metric (layer F.Cu) (at 27.8638 82.6262 270)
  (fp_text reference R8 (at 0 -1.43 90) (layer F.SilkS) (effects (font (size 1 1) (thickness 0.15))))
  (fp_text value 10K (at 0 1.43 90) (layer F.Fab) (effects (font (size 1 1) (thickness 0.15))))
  (pad 2 smd roundrect (at 0.7875 0 270) (size 0.875 0.95) (layers F.Cu F.Paste F.Mask) (roundrect_rratio 0.25) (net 43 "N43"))
  (pad 1 smd roundrect (at -0.7875 0 270) (size 0.875 0.95) (layers F.Cu F.Paste F.Mask) (roundrect_rratio 0.25) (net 31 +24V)))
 (gr_line (start 93 28) (end 16 28) (layer Edge.Cuts) (width 0.05))
 (gr_line (start 16 92.5) (end 93 92.5) (layer Edge.Cuts) (width 0.05))
 (via (at 62.0776 45.6692) (size 3) (drill 1) (layers F.Cu B.Cu) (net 2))
 (segment (start 62.0268 45.72) (end 62.0776 45.6692) (width 0.3) (layer F.Cu) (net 2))
 (segment (start 59.69 45.72) (end 62.0268 45.72) (width 0.3) (layer F.Cu) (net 2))
 (via (at 62.450301 71.589838) (size 3) (drill 1) (layers F.Cu B.Cu) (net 2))
 (segment (start 62.0776 71.217137) (end 62.450301 71.589838) (width 0.3) (layer B.Cu) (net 2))
 (segment (start 62.0776 45.6692) (end 62.0776 71.217137) (width 0.3) (layer B.Cu) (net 2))
 (segment (start 65.900362 71.589838) (end 66.04 71.4502) (width 0.3) (layer F.Cu) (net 2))
 (segment (start 62.450301 71.589838) (end 65.900362 71.589838) (width 0.3) (layer F.Cu) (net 2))
 (segment (start 66.04 53.9502) (end 66.04 53.213) (width 0.3) (layer F.Cu) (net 3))
 (segment (start 63.627 50.8) (end 59.69 50.8) (width 0.3) (layer F.Cu) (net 3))
 (segment (start 66.04 53.213) (end 63.627 50.8) (width 0.3) (layer F.Cu) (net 3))
 (segment (start 44.45 66.04) (end 40.95759 69.53241) (width 0.3) (layer F.Cu) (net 21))
 (segment (start 40.95759 70.941024) (end 40.234414 71.6642) (width 0.3) (layer F.Cu) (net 21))
 (segment (start 40.95759 69.53241) (end 40.95759 70.941024) (width 0.3) (layer F.Cu) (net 21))
 (segment (start 40.234414 71.6642) (end 39.1414 71.6642) (width 0.3) (layer F.Cu) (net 21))
 (segment (start 44.45 68.58) (end 40.76641 72.26359) (width 0.3) (layer F.Cu) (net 23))
 (segment (start 40.76641 72.53919) (end 39.1414 74.1642) (width 0.3) (layer F.Cu) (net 23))
 (segment (start 40.76641 72.26359) (end 40.76641 72.53919) (width 0.3) (layer F.Cu) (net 23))
 (segment (start 42.1456 73.66) (end 39.1414 76.6642) (width 0.3) (layer F.Cu) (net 26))
 (segment (start 44.45 73.66) (end 42.1456 73.66) (width 0.3) (layer F.Cu) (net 26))
 (segment (start 42.1056 76.2) (end 39.1414 79.1642) (width 0.3) (layer F.Cu) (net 27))
 (segment (start 44.45 76.2) (end 42.1056 76.2) (width 0.3) (layer F.Cu) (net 27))
 (segment (start 42.0656 78.74) (end 39.1414 81.6642) (width 0.3) (layer F.Cu) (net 29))
 (segment (start 44.45 78.74) (end 42.0656 78.74) (width 0.3) (layer F.Cu) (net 29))
 (segment (start 54.2658 84.1642) (end 59.69 78.74) (width 0.3) (layer F.Cu) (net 30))
 (segment (start 39.1414 84.1642) (end 54.2658 84.1642) (width 0.3) (layer F.Cu) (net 30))
 (segment (start 62.9298 53.34) (end 66.04 56.4502) (width 0.3) (layer F.Cu) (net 22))
 (segment (start 59.69 53.34) (end 62.9298 53.34) (width 0.3) (layer F.Cu) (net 22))
 (segment (start 62.9698 55.88) (end 66.04 58.9502) (width 0.3) (layer F.Cu) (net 20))
 (segment (start 59.69 55.88) (end 62.9698 55.88) (width 0.3) (layer F.Cu) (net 20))
 (segment (start 63.9902 63.5) (end 66.04 61.4502) (width 0.3) (layer F.Cu) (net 14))
 (segment (start 59.69 63.5) (end 63.9902 63.5) (width 0.3) (layer F.Cu) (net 14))
 (segment (start 63.9502 66.04) (end 66.04 63.9502) (width 0.3) (layer F.Cu) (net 12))
 (segment (start 59.69 66.04) (end 63.9502 66.04) (width 0.3) (layer F.Cu) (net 12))
 (segment (start 59.69 68.58) (end 60.119811 68.150189) (width 0.3) (layer F.Cu) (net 10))
 (segment (start 60.119811 68.150189) (end 64.340011 68.150189) (width 0.3) (layer F.Cu) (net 10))
 (segment (start 64.340011 68.150189) (end 66.04 66.4502) (width 0.3) (layer F.Cu) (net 10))
 (segment (start 61.8598 68.9502) (end 59.69 71.12) (width 0.3) (layer F.Cu) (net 9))
 (segment (start 66.04 68.9502) (end 61.8598 68.9502) (width 0.3) (layer F.Cu) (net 9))
 (segment (start 43.6156 57.5856) (end 44.45 58.42) (width 0.3) (layer F.Cu) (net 15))
 (segment (start 38.2778 57.5856) (end 43.6156 57.5856) (width 0.3) (layer F.Cu) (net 15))
 (segment (start 42.7044 55.0856) (end 44.45 53.34) (width 0.3) (layer F.Cu) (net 11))
 (segment (start 38.2778 55.0856) (end 42.7044 55.0856) (width 0.3) (layer F.Cu) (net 11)))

